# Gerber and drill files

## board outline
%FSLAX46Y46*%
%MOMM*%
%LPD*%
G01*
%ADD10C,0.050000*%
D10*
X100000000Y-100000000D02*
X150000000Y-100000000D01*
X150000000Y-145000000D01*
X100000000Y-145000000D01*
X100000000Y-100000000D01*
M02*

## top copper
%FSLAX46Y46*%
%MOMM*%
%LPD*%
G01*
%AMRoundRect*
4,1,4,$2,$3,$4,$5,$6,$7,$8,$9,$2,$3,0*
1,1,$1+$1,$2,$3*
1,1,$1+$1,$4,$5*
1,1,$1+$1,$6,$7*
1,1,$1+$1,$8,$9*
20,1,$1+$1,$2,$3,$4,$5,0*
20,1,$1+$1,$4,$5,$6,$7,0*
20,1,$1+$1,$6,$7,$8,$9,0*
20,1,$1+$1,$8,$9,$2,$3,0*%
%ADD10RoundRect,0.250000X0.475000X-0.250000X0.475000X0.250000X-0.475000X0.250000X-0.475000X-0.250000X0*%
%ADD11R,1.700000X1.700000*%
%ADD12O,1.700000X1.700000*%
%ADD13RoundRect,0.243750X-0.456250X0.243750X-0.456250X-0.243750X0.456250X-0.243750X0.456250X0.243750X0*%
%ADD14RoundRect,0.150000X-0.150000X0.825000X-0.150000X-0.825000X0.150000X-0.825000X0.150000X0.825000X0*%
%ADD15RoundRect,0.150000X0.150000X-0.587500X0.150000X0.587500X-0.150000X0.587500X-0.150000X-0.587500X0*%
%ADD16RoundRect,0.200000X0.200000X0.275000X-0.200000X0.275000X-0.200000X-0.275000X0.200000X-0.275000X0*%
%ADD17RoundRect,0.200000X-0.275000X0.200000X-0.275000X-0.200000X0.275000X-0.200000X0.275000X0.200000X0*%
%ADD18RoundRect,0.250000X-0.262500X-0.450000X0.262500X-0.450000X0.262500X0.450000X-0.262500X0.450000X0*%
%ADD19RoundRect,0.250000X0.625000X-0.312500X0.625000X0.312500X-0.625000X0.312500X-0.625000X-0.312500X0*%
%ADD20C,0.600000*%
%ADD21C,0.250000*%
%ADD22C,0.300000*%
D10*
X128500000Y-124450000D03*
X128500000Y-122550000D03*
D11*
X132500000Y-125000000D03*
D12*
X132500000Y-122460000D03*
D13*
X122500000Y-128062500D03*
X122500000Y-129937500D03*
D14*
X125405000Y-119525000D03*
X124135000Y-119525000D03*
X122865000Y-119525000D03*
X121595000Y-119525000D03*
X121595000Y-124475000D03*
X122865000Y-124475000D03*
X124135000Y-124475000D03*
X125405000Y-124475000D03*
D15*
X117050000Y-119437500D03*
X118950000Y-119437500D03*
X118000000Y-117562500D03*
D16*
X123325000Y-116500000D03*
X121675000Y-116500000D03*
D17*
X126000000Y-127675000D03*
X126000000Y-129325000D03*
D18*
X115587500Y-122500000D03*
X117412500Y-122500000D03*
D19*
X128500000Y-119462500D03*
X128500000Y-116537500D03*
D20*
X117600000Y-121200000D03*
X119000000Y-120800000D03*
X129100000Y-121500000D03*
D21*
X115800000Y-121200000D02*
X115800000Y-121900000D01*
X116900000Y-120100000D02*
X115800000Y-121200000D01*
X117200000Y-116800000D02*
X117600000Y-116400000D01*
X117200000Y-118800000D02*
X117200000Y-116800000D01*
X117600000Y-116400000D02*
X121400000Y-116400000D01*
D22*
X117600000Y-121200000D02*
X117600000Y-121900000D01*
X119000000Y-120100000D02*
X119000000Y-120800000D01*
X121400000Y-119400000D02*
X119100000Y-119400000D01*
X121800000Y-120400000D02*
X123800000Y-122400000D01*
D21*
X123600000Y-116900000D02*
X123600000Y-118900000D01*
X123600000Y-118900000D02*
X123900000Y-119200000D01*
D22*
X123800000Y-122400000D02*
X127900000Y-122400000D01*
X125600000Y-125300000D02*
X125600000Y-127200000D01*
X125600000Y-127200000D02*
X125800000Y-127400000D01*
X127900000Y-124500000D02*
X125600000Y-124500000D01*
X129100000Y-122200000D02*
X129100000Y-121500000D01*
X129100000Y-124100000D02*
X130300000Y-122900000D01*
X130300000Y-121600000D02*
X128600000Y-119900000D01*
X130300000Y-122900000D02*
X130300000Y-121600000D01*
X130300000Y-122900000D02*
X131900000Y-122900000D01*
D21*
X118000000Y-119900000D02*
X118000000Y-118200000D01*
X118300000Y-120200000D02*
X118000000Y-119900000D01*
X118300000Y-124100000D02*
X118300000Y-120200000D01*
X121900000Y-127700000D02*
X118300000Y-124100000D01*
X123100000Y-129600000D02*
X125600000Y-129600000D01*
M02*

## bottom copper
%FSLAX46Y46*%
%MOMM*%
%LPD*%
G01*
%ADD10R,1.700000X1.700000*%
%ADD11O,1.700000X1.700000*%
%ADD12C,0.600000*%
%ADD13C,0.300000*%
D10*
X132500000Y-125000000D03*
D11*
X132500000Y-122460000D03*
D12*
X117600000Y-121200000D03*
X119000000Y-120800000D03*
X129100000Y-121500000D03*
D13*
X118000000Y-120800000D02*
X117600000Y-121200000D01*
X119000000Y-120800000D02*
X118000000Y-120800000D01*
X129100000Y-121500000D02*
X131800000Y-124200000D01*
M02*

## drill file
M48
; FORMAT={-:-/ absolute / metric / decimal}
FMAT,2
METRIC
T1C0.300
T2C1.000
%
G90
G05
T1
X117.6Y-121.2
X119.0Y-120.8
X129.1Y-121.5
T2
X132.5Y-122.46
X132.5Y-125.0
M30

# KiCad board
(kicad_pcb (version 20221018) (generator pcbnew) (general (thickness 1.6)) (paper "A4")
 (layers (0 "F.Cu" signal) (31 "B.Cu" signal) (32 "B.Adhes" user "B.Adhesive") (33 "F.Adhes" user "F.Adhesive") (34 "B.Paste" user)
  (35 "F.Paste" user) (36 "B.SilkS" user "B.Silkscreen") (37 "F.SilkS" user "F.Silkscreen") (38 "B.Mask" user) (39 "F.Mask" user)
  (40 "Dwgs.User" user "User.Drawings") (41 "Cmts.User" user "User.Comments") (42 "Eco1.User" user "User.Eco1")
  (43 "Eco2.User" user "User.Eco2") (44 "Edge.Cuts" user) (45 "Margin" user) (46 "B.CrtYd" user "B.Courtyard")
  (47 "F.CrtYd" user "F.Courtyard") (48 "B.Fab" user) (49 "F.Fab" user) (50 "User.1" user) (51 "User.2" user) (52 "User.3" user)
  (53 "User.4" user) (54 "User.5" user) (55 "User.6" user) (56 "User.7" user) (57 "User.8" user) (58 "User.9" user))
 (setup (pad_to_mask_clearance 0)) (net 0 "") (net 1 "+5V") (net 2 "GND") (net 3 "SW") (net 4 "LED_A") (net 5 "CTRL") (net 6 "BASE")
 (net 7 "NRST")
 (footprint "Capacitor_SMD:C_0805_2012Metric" (layer "F.Cu") (at 128.5 123.5 90)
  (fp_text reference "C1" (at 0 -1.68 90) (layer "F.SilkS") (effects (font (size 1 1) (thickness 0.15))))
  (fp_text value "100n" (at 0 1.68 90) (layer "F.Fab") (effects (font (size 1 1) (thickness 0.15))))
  (pad "1" smd roundrect (at -0.95 0 90) (size 1 1.45) (layers "F.Cu" "F.Paste" "F.Mask") (roundrect_rratio 0.25) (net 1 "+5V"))
  (pad "2" smd roundrect (at 0.95 0 90) (size 1 1.45) (layers "F.Cu" "F.Paste" "F.Mask") (roundrect_rratio 0.25) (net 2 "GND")))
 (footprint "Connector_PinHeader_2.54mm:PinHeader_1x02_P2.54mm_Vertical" (layer "F.Cu") (at 132.5 125 180)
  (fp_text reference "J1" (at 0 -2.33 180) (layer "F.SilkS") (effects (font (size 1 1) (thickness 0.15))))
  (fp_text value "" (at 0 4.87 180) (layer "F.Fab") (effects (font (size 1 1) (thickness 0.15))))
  (pad "1" thru_hole rect (at 0 0 180) (size 1.7 1.7) (drill 1) (layers "*.Cu" "*.Mask") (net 2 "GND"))
  (pad "2" thru_hole oval (at 0 2.54 180) (size 1.7 1.7) (drill 1) (layers "*.Cu" "*.Mask") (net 1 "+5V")))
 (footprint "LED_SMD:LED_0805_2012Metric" (layer "F.Cu") (at 122.5 129 -90)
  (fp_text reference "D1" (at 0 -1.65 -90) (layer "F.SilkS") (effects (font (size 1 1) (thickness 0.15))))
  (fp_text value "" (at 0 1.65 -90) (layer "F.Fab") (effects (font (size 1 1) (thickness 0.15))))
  (pad "1" smd roundrect (at -0.9375 0 270) (size 0.975 1.4) (layers "F.Cu" "F.Paste" "F.Mask") (roundrect_rratio 0.25) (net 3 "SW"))
  (pad "2" smd roundrect (at 0.9375 0 270) (size 0.975 1.4) (layers "F.Cu" "F.Paste" "F.Mask") (roundrect_rratio 0.25) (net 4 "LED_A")))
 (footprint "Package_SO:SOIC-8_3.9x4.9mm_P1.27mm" (layer "F.Cu") (at 123.5 122 -90)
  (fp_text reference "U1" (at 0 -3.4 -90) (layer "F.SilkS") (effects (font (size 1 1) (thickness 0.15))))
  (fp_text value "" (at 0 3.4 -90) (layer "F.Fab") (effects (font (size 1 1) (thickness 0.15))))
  (pad "1" smd roundrect (at -2.475 -1.905 270) (size 1.95 0.6) (layers "F.Cu" "F.Paste" "F.Mask") (roundrect_rratio 0.25))
  (pad "2" smd roundrect (at -2.475 -0.635 270) (size 1.95 0.6) (layers "F.Cu" "F.Paste" "F.Mask") (roundrect_rratio 0.25) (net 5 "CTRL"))
  (pad "3" smd roundrect (at -2.475 0.635 270) (size 1.95 0.6) (layers "F.Cu" "F.Paste" "F.Mask") (roundrect_rratio 0.25))
  (pad "4" smd roundrect (at -2.475 1.905 270) (size 1.95 0.6) (layers "F.Cu" "F.Paste" "F.Mask") (roundrect_rratio 0.25) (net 2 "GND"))
  (pad "5" smd roundrect (at 2.475 1.905 270) (size 1.95 0.6) (layers "F.Cu" "F.Paste" "F.Mask") (roundrect_rratio 0.25))
  (pad "6" smd roundrect (at 2.475 0.635 270) (size 1.95 0.6) (layers "F.Cu" "F.Paste" "F.Mask") (roundrect_rratio 0.25))
  (pad "7" smd roundrect (at 2.475 -0.635 270) (size 1.95 0.6) (layers "F.Cu" "F.Paste" "F.Mask") (roundrect_rratio 0.25))
  (pad "8" smd roundrect (at 2.475 -1.905 270) (size 1.95 0.6) (layers "F.Cu" "F.Paste" "F.Mask") (roundrect_rratio 0.25) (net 1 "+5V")))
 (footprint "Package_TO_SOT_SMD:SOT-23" (layer "F.Cu") (at 118 118.5 90)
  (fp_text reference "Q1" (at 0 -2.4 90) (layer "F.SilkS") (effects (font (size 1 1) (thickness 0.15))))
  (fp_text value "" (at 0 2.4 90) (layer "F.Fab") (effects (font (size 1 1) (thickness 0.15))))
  (pad "1" smd roundrect (at -0.9375 -0.95 90) (size 1.475 0.6) (layers "F.Cu" "F.Paste" "F.Mask") (roundrect_rratio 0.25) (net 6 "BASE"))
  (pad "2" smd roundrect (at -0.9375 0.95 90) (size 1.475 0.6) (layers "F.Cu" "F.Paste" "F.Mask") (roundrect_rratio 0.25) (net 2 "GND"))
  (pad "3" smd roundrect (at 0.9375 0 90) (size 1.475 0.6) (layers "F.Cu" "F.Paste" "F.Mask") (roundrect_rratio 0.25) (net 3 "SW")))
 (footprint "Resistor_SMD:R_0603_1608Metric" (layer "F.Cu") (at 122.5 116.5 180)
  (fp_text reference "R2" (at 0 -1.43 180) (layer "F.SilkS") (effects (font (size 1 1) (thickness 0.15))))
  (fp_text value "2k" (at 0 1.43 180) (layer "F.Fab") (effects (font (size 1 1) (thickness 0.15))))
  (pad "1" smd roundrect (at -0.825 0 180) (size 0.8 0.95) (layers "F.Cu" "F.Paste" "F.Mask") (roundrect_rratio 0.25) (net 5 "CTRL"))
  (pad "2" smd roundrect (at 0.825 0 180) (size 0.8 0.95) (layers "F.Cu" "F.Paste" "F.Mask") (roundrect_rratio 0.25) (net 6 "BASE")))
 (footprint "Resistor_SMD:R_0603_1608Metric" (layer "F.Cu") (at 126 128.5 -90)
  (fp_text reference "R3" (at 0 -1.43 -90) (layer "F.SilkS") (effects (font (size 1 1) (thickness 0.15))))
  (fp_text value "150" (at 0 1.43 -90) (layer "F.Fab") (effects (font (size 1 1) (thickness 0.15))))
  (pad "1" smd roundrect (at -0.825 0 270) (size 0.8 0.95) (layers "F.Cu" "F.Paste" "F.Mask") (roundrect_rratio 0.25) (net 1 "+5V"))
  (pad "2" smd roundrect (at 0.825 0 270) (size 0.8 0.95) (layers "F.Cu" "F.Paste" "F.Mask") (roundrect_rratio 0.25) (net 4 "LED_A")))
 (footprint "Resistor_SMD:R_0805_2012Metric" (layer "F.Cu") (at 116.5 122.5)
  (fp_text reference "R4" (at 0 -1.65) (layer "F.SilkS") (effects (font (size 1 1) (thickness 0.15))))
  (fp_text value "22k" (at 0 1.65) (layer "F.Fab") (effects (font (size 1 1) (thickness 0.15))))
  (pad "1" smd roundrect (at -0.9125 0) (size 1.025 1.4) (layers "F.Cu" "F.Paste" "F.Mask") (roundrect_rratio 0.243902) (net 6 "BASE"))
  (pad "2" smd roundrect (at 0.9125 0) (size 1.025 1.4) (layers "F.Cu" "F.Paste" "F.Mask") (roundrect_rratio 0.243902) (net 2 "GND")))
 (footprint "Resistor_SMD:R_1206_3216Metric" (layer "F.Cu") (at 128.5 118 90)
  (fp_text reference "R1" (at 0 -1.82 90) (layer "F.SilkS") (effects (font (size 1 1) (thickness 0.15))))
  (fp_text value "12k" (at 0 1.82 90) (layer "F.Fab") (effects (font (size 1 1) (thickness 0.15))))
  (pad "1" smd roundrect (at -1.4625 0 90) (size 1.125 1.75) (layers "F.Cu" "F.Paste" "F.Mask") (roundrect_rratio 0.222222) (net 1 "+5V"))
  (pad "2" smd roundrect (at 1.4625 0 90) (size 1.125 1.75) (layers "F.Cu" "F.Paste" "F.Mask") (roundrect_rratio 0.222222) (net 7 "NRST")))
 (gr_rect (start 100 100) (end 150 145) (stroke (width 0.05) (type default)) (fill none) (layer "Edge.Cuts"))
 (segment (start 115.8 121.2) (end 115.8 121.9) (width 0.25) (layer "F.Cu") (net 6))
 (segment (start 116.9 120.1) (end 115.8 121.2) (width 0.25) (layer "F.Cu") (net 6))
 (segment (start 117.2 116.8) (end 117.6 116.4) (width 0.25) (layer "F.Cu") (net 6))
 (segment (start 117.2 118.8) (end 117.2 116.8) (width 0.25) (layer "F.Cu") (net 6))
 (segment (start 117.6 116.4) (end 121.4 116.4) (width 0.25) (layer "F.Cu") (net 6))
 (segment (start 117.6 121.2) (end 117.6 121.9) (width 0.3) (layer "F.Cu") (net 2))
 (segment (start 119 120.1) (end 119 120.8) (width 0.3) (layer "F.Cu") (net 2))
 (segment (start 121.4 119.4) (end 119.1 119.4) (width 0.3) (layer "F.Cu") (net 2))
 (segment (start 121.8 120.4) (end 123.8 122.4) (width 0.3) (layer "F.Cu") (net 2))
 (segment (start 123.6 116.9) (end 123.6 118.9) (width 0.25) (layer "F.Cu") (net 5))
 (segment (start 123.6 118.9) (end 123.9 119.2) (width 0.25) (layer "F.Cu") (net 5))
 (segment (start 123.8 122.4) (end 127.9 122.4) (width 0.3) (layer "F.Cu") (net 2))
 (segment (start 125.6 125.3) (end 125.6 127.2) (width 0.3) (layer "F.Cu") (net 1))
 (segment (start 125.6 127.2) (end 125.8 127.4) (width 0.3) (layer "F.Cu") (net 1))
 (segment (start 127.9 124.5) (end 125.6 124.5) (width 0.3) (layer "F.Cu") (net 1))
 (segment (start 129.1 122.2) (end 129.1 121.5) (width 0.3) (layer "F.Cu") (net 2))
 (segment (start 129.1 124.1) (end 130.3 122.9) (width 0.3) (layer "F.Cu") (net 1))
 (segment (start 130.3 121.6) (end 128.6 119.9) (width 0.3) (layer "F.Cu") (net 1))
 (segment (start 130.3 122.9) (end 130.3 121.6) (width 0.3) (layer "F.Cu") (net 1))
 (segment (start 130.3 122.9) (end 131.9 122.9) (width 0.3) (layer "F.Cu") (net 1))
 (via (at 117.6 121.2) (size 0.6) (drill 0.3) (layers "F.Cu" "B.Cu") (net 2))
 (via (at 119 120.8) (size 0.6) (drill 0.3) (layers "F.Cu" "B.Cu") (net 2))
 (via (at 129.1 121.5) (size 0.6) (drill 0.3) (layers "F.Cu" "B.Cu") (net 2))
 (segment (start 118 119.9) (end 118 118.2) (width 0.25) (layer "F.Cu") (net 3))
 (segment (start 118 120.8) (end 117.6 121.2) (width 0.3) (layer "B.Cu") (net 2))
 (segment (start 118.3 120.2) (end 118 119.9) (width 0.25) (layer "F.Cu") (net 3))
 (segment (start 118.3 124.1) (end 118.3 120.2) (width 0.25) (layer "F.Cu") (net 3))
 (segment (start 119 120.8) (end 118 120.8) (width 0.3) (layer "B.Cu") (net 2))
 (segment (start 121.9 127.7) (end 118.3 124.1) (width 0.25) (layer "F.Cu") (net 3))
 (segment (start 123.1 129.6) (end 125.6 129.6) (width 0.25) (layer "F.Cu") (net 4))
 (segment (start 129.1 121.5) (end 131.8 124.2) (width 0.3) (layer "B.Cu") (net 2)))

